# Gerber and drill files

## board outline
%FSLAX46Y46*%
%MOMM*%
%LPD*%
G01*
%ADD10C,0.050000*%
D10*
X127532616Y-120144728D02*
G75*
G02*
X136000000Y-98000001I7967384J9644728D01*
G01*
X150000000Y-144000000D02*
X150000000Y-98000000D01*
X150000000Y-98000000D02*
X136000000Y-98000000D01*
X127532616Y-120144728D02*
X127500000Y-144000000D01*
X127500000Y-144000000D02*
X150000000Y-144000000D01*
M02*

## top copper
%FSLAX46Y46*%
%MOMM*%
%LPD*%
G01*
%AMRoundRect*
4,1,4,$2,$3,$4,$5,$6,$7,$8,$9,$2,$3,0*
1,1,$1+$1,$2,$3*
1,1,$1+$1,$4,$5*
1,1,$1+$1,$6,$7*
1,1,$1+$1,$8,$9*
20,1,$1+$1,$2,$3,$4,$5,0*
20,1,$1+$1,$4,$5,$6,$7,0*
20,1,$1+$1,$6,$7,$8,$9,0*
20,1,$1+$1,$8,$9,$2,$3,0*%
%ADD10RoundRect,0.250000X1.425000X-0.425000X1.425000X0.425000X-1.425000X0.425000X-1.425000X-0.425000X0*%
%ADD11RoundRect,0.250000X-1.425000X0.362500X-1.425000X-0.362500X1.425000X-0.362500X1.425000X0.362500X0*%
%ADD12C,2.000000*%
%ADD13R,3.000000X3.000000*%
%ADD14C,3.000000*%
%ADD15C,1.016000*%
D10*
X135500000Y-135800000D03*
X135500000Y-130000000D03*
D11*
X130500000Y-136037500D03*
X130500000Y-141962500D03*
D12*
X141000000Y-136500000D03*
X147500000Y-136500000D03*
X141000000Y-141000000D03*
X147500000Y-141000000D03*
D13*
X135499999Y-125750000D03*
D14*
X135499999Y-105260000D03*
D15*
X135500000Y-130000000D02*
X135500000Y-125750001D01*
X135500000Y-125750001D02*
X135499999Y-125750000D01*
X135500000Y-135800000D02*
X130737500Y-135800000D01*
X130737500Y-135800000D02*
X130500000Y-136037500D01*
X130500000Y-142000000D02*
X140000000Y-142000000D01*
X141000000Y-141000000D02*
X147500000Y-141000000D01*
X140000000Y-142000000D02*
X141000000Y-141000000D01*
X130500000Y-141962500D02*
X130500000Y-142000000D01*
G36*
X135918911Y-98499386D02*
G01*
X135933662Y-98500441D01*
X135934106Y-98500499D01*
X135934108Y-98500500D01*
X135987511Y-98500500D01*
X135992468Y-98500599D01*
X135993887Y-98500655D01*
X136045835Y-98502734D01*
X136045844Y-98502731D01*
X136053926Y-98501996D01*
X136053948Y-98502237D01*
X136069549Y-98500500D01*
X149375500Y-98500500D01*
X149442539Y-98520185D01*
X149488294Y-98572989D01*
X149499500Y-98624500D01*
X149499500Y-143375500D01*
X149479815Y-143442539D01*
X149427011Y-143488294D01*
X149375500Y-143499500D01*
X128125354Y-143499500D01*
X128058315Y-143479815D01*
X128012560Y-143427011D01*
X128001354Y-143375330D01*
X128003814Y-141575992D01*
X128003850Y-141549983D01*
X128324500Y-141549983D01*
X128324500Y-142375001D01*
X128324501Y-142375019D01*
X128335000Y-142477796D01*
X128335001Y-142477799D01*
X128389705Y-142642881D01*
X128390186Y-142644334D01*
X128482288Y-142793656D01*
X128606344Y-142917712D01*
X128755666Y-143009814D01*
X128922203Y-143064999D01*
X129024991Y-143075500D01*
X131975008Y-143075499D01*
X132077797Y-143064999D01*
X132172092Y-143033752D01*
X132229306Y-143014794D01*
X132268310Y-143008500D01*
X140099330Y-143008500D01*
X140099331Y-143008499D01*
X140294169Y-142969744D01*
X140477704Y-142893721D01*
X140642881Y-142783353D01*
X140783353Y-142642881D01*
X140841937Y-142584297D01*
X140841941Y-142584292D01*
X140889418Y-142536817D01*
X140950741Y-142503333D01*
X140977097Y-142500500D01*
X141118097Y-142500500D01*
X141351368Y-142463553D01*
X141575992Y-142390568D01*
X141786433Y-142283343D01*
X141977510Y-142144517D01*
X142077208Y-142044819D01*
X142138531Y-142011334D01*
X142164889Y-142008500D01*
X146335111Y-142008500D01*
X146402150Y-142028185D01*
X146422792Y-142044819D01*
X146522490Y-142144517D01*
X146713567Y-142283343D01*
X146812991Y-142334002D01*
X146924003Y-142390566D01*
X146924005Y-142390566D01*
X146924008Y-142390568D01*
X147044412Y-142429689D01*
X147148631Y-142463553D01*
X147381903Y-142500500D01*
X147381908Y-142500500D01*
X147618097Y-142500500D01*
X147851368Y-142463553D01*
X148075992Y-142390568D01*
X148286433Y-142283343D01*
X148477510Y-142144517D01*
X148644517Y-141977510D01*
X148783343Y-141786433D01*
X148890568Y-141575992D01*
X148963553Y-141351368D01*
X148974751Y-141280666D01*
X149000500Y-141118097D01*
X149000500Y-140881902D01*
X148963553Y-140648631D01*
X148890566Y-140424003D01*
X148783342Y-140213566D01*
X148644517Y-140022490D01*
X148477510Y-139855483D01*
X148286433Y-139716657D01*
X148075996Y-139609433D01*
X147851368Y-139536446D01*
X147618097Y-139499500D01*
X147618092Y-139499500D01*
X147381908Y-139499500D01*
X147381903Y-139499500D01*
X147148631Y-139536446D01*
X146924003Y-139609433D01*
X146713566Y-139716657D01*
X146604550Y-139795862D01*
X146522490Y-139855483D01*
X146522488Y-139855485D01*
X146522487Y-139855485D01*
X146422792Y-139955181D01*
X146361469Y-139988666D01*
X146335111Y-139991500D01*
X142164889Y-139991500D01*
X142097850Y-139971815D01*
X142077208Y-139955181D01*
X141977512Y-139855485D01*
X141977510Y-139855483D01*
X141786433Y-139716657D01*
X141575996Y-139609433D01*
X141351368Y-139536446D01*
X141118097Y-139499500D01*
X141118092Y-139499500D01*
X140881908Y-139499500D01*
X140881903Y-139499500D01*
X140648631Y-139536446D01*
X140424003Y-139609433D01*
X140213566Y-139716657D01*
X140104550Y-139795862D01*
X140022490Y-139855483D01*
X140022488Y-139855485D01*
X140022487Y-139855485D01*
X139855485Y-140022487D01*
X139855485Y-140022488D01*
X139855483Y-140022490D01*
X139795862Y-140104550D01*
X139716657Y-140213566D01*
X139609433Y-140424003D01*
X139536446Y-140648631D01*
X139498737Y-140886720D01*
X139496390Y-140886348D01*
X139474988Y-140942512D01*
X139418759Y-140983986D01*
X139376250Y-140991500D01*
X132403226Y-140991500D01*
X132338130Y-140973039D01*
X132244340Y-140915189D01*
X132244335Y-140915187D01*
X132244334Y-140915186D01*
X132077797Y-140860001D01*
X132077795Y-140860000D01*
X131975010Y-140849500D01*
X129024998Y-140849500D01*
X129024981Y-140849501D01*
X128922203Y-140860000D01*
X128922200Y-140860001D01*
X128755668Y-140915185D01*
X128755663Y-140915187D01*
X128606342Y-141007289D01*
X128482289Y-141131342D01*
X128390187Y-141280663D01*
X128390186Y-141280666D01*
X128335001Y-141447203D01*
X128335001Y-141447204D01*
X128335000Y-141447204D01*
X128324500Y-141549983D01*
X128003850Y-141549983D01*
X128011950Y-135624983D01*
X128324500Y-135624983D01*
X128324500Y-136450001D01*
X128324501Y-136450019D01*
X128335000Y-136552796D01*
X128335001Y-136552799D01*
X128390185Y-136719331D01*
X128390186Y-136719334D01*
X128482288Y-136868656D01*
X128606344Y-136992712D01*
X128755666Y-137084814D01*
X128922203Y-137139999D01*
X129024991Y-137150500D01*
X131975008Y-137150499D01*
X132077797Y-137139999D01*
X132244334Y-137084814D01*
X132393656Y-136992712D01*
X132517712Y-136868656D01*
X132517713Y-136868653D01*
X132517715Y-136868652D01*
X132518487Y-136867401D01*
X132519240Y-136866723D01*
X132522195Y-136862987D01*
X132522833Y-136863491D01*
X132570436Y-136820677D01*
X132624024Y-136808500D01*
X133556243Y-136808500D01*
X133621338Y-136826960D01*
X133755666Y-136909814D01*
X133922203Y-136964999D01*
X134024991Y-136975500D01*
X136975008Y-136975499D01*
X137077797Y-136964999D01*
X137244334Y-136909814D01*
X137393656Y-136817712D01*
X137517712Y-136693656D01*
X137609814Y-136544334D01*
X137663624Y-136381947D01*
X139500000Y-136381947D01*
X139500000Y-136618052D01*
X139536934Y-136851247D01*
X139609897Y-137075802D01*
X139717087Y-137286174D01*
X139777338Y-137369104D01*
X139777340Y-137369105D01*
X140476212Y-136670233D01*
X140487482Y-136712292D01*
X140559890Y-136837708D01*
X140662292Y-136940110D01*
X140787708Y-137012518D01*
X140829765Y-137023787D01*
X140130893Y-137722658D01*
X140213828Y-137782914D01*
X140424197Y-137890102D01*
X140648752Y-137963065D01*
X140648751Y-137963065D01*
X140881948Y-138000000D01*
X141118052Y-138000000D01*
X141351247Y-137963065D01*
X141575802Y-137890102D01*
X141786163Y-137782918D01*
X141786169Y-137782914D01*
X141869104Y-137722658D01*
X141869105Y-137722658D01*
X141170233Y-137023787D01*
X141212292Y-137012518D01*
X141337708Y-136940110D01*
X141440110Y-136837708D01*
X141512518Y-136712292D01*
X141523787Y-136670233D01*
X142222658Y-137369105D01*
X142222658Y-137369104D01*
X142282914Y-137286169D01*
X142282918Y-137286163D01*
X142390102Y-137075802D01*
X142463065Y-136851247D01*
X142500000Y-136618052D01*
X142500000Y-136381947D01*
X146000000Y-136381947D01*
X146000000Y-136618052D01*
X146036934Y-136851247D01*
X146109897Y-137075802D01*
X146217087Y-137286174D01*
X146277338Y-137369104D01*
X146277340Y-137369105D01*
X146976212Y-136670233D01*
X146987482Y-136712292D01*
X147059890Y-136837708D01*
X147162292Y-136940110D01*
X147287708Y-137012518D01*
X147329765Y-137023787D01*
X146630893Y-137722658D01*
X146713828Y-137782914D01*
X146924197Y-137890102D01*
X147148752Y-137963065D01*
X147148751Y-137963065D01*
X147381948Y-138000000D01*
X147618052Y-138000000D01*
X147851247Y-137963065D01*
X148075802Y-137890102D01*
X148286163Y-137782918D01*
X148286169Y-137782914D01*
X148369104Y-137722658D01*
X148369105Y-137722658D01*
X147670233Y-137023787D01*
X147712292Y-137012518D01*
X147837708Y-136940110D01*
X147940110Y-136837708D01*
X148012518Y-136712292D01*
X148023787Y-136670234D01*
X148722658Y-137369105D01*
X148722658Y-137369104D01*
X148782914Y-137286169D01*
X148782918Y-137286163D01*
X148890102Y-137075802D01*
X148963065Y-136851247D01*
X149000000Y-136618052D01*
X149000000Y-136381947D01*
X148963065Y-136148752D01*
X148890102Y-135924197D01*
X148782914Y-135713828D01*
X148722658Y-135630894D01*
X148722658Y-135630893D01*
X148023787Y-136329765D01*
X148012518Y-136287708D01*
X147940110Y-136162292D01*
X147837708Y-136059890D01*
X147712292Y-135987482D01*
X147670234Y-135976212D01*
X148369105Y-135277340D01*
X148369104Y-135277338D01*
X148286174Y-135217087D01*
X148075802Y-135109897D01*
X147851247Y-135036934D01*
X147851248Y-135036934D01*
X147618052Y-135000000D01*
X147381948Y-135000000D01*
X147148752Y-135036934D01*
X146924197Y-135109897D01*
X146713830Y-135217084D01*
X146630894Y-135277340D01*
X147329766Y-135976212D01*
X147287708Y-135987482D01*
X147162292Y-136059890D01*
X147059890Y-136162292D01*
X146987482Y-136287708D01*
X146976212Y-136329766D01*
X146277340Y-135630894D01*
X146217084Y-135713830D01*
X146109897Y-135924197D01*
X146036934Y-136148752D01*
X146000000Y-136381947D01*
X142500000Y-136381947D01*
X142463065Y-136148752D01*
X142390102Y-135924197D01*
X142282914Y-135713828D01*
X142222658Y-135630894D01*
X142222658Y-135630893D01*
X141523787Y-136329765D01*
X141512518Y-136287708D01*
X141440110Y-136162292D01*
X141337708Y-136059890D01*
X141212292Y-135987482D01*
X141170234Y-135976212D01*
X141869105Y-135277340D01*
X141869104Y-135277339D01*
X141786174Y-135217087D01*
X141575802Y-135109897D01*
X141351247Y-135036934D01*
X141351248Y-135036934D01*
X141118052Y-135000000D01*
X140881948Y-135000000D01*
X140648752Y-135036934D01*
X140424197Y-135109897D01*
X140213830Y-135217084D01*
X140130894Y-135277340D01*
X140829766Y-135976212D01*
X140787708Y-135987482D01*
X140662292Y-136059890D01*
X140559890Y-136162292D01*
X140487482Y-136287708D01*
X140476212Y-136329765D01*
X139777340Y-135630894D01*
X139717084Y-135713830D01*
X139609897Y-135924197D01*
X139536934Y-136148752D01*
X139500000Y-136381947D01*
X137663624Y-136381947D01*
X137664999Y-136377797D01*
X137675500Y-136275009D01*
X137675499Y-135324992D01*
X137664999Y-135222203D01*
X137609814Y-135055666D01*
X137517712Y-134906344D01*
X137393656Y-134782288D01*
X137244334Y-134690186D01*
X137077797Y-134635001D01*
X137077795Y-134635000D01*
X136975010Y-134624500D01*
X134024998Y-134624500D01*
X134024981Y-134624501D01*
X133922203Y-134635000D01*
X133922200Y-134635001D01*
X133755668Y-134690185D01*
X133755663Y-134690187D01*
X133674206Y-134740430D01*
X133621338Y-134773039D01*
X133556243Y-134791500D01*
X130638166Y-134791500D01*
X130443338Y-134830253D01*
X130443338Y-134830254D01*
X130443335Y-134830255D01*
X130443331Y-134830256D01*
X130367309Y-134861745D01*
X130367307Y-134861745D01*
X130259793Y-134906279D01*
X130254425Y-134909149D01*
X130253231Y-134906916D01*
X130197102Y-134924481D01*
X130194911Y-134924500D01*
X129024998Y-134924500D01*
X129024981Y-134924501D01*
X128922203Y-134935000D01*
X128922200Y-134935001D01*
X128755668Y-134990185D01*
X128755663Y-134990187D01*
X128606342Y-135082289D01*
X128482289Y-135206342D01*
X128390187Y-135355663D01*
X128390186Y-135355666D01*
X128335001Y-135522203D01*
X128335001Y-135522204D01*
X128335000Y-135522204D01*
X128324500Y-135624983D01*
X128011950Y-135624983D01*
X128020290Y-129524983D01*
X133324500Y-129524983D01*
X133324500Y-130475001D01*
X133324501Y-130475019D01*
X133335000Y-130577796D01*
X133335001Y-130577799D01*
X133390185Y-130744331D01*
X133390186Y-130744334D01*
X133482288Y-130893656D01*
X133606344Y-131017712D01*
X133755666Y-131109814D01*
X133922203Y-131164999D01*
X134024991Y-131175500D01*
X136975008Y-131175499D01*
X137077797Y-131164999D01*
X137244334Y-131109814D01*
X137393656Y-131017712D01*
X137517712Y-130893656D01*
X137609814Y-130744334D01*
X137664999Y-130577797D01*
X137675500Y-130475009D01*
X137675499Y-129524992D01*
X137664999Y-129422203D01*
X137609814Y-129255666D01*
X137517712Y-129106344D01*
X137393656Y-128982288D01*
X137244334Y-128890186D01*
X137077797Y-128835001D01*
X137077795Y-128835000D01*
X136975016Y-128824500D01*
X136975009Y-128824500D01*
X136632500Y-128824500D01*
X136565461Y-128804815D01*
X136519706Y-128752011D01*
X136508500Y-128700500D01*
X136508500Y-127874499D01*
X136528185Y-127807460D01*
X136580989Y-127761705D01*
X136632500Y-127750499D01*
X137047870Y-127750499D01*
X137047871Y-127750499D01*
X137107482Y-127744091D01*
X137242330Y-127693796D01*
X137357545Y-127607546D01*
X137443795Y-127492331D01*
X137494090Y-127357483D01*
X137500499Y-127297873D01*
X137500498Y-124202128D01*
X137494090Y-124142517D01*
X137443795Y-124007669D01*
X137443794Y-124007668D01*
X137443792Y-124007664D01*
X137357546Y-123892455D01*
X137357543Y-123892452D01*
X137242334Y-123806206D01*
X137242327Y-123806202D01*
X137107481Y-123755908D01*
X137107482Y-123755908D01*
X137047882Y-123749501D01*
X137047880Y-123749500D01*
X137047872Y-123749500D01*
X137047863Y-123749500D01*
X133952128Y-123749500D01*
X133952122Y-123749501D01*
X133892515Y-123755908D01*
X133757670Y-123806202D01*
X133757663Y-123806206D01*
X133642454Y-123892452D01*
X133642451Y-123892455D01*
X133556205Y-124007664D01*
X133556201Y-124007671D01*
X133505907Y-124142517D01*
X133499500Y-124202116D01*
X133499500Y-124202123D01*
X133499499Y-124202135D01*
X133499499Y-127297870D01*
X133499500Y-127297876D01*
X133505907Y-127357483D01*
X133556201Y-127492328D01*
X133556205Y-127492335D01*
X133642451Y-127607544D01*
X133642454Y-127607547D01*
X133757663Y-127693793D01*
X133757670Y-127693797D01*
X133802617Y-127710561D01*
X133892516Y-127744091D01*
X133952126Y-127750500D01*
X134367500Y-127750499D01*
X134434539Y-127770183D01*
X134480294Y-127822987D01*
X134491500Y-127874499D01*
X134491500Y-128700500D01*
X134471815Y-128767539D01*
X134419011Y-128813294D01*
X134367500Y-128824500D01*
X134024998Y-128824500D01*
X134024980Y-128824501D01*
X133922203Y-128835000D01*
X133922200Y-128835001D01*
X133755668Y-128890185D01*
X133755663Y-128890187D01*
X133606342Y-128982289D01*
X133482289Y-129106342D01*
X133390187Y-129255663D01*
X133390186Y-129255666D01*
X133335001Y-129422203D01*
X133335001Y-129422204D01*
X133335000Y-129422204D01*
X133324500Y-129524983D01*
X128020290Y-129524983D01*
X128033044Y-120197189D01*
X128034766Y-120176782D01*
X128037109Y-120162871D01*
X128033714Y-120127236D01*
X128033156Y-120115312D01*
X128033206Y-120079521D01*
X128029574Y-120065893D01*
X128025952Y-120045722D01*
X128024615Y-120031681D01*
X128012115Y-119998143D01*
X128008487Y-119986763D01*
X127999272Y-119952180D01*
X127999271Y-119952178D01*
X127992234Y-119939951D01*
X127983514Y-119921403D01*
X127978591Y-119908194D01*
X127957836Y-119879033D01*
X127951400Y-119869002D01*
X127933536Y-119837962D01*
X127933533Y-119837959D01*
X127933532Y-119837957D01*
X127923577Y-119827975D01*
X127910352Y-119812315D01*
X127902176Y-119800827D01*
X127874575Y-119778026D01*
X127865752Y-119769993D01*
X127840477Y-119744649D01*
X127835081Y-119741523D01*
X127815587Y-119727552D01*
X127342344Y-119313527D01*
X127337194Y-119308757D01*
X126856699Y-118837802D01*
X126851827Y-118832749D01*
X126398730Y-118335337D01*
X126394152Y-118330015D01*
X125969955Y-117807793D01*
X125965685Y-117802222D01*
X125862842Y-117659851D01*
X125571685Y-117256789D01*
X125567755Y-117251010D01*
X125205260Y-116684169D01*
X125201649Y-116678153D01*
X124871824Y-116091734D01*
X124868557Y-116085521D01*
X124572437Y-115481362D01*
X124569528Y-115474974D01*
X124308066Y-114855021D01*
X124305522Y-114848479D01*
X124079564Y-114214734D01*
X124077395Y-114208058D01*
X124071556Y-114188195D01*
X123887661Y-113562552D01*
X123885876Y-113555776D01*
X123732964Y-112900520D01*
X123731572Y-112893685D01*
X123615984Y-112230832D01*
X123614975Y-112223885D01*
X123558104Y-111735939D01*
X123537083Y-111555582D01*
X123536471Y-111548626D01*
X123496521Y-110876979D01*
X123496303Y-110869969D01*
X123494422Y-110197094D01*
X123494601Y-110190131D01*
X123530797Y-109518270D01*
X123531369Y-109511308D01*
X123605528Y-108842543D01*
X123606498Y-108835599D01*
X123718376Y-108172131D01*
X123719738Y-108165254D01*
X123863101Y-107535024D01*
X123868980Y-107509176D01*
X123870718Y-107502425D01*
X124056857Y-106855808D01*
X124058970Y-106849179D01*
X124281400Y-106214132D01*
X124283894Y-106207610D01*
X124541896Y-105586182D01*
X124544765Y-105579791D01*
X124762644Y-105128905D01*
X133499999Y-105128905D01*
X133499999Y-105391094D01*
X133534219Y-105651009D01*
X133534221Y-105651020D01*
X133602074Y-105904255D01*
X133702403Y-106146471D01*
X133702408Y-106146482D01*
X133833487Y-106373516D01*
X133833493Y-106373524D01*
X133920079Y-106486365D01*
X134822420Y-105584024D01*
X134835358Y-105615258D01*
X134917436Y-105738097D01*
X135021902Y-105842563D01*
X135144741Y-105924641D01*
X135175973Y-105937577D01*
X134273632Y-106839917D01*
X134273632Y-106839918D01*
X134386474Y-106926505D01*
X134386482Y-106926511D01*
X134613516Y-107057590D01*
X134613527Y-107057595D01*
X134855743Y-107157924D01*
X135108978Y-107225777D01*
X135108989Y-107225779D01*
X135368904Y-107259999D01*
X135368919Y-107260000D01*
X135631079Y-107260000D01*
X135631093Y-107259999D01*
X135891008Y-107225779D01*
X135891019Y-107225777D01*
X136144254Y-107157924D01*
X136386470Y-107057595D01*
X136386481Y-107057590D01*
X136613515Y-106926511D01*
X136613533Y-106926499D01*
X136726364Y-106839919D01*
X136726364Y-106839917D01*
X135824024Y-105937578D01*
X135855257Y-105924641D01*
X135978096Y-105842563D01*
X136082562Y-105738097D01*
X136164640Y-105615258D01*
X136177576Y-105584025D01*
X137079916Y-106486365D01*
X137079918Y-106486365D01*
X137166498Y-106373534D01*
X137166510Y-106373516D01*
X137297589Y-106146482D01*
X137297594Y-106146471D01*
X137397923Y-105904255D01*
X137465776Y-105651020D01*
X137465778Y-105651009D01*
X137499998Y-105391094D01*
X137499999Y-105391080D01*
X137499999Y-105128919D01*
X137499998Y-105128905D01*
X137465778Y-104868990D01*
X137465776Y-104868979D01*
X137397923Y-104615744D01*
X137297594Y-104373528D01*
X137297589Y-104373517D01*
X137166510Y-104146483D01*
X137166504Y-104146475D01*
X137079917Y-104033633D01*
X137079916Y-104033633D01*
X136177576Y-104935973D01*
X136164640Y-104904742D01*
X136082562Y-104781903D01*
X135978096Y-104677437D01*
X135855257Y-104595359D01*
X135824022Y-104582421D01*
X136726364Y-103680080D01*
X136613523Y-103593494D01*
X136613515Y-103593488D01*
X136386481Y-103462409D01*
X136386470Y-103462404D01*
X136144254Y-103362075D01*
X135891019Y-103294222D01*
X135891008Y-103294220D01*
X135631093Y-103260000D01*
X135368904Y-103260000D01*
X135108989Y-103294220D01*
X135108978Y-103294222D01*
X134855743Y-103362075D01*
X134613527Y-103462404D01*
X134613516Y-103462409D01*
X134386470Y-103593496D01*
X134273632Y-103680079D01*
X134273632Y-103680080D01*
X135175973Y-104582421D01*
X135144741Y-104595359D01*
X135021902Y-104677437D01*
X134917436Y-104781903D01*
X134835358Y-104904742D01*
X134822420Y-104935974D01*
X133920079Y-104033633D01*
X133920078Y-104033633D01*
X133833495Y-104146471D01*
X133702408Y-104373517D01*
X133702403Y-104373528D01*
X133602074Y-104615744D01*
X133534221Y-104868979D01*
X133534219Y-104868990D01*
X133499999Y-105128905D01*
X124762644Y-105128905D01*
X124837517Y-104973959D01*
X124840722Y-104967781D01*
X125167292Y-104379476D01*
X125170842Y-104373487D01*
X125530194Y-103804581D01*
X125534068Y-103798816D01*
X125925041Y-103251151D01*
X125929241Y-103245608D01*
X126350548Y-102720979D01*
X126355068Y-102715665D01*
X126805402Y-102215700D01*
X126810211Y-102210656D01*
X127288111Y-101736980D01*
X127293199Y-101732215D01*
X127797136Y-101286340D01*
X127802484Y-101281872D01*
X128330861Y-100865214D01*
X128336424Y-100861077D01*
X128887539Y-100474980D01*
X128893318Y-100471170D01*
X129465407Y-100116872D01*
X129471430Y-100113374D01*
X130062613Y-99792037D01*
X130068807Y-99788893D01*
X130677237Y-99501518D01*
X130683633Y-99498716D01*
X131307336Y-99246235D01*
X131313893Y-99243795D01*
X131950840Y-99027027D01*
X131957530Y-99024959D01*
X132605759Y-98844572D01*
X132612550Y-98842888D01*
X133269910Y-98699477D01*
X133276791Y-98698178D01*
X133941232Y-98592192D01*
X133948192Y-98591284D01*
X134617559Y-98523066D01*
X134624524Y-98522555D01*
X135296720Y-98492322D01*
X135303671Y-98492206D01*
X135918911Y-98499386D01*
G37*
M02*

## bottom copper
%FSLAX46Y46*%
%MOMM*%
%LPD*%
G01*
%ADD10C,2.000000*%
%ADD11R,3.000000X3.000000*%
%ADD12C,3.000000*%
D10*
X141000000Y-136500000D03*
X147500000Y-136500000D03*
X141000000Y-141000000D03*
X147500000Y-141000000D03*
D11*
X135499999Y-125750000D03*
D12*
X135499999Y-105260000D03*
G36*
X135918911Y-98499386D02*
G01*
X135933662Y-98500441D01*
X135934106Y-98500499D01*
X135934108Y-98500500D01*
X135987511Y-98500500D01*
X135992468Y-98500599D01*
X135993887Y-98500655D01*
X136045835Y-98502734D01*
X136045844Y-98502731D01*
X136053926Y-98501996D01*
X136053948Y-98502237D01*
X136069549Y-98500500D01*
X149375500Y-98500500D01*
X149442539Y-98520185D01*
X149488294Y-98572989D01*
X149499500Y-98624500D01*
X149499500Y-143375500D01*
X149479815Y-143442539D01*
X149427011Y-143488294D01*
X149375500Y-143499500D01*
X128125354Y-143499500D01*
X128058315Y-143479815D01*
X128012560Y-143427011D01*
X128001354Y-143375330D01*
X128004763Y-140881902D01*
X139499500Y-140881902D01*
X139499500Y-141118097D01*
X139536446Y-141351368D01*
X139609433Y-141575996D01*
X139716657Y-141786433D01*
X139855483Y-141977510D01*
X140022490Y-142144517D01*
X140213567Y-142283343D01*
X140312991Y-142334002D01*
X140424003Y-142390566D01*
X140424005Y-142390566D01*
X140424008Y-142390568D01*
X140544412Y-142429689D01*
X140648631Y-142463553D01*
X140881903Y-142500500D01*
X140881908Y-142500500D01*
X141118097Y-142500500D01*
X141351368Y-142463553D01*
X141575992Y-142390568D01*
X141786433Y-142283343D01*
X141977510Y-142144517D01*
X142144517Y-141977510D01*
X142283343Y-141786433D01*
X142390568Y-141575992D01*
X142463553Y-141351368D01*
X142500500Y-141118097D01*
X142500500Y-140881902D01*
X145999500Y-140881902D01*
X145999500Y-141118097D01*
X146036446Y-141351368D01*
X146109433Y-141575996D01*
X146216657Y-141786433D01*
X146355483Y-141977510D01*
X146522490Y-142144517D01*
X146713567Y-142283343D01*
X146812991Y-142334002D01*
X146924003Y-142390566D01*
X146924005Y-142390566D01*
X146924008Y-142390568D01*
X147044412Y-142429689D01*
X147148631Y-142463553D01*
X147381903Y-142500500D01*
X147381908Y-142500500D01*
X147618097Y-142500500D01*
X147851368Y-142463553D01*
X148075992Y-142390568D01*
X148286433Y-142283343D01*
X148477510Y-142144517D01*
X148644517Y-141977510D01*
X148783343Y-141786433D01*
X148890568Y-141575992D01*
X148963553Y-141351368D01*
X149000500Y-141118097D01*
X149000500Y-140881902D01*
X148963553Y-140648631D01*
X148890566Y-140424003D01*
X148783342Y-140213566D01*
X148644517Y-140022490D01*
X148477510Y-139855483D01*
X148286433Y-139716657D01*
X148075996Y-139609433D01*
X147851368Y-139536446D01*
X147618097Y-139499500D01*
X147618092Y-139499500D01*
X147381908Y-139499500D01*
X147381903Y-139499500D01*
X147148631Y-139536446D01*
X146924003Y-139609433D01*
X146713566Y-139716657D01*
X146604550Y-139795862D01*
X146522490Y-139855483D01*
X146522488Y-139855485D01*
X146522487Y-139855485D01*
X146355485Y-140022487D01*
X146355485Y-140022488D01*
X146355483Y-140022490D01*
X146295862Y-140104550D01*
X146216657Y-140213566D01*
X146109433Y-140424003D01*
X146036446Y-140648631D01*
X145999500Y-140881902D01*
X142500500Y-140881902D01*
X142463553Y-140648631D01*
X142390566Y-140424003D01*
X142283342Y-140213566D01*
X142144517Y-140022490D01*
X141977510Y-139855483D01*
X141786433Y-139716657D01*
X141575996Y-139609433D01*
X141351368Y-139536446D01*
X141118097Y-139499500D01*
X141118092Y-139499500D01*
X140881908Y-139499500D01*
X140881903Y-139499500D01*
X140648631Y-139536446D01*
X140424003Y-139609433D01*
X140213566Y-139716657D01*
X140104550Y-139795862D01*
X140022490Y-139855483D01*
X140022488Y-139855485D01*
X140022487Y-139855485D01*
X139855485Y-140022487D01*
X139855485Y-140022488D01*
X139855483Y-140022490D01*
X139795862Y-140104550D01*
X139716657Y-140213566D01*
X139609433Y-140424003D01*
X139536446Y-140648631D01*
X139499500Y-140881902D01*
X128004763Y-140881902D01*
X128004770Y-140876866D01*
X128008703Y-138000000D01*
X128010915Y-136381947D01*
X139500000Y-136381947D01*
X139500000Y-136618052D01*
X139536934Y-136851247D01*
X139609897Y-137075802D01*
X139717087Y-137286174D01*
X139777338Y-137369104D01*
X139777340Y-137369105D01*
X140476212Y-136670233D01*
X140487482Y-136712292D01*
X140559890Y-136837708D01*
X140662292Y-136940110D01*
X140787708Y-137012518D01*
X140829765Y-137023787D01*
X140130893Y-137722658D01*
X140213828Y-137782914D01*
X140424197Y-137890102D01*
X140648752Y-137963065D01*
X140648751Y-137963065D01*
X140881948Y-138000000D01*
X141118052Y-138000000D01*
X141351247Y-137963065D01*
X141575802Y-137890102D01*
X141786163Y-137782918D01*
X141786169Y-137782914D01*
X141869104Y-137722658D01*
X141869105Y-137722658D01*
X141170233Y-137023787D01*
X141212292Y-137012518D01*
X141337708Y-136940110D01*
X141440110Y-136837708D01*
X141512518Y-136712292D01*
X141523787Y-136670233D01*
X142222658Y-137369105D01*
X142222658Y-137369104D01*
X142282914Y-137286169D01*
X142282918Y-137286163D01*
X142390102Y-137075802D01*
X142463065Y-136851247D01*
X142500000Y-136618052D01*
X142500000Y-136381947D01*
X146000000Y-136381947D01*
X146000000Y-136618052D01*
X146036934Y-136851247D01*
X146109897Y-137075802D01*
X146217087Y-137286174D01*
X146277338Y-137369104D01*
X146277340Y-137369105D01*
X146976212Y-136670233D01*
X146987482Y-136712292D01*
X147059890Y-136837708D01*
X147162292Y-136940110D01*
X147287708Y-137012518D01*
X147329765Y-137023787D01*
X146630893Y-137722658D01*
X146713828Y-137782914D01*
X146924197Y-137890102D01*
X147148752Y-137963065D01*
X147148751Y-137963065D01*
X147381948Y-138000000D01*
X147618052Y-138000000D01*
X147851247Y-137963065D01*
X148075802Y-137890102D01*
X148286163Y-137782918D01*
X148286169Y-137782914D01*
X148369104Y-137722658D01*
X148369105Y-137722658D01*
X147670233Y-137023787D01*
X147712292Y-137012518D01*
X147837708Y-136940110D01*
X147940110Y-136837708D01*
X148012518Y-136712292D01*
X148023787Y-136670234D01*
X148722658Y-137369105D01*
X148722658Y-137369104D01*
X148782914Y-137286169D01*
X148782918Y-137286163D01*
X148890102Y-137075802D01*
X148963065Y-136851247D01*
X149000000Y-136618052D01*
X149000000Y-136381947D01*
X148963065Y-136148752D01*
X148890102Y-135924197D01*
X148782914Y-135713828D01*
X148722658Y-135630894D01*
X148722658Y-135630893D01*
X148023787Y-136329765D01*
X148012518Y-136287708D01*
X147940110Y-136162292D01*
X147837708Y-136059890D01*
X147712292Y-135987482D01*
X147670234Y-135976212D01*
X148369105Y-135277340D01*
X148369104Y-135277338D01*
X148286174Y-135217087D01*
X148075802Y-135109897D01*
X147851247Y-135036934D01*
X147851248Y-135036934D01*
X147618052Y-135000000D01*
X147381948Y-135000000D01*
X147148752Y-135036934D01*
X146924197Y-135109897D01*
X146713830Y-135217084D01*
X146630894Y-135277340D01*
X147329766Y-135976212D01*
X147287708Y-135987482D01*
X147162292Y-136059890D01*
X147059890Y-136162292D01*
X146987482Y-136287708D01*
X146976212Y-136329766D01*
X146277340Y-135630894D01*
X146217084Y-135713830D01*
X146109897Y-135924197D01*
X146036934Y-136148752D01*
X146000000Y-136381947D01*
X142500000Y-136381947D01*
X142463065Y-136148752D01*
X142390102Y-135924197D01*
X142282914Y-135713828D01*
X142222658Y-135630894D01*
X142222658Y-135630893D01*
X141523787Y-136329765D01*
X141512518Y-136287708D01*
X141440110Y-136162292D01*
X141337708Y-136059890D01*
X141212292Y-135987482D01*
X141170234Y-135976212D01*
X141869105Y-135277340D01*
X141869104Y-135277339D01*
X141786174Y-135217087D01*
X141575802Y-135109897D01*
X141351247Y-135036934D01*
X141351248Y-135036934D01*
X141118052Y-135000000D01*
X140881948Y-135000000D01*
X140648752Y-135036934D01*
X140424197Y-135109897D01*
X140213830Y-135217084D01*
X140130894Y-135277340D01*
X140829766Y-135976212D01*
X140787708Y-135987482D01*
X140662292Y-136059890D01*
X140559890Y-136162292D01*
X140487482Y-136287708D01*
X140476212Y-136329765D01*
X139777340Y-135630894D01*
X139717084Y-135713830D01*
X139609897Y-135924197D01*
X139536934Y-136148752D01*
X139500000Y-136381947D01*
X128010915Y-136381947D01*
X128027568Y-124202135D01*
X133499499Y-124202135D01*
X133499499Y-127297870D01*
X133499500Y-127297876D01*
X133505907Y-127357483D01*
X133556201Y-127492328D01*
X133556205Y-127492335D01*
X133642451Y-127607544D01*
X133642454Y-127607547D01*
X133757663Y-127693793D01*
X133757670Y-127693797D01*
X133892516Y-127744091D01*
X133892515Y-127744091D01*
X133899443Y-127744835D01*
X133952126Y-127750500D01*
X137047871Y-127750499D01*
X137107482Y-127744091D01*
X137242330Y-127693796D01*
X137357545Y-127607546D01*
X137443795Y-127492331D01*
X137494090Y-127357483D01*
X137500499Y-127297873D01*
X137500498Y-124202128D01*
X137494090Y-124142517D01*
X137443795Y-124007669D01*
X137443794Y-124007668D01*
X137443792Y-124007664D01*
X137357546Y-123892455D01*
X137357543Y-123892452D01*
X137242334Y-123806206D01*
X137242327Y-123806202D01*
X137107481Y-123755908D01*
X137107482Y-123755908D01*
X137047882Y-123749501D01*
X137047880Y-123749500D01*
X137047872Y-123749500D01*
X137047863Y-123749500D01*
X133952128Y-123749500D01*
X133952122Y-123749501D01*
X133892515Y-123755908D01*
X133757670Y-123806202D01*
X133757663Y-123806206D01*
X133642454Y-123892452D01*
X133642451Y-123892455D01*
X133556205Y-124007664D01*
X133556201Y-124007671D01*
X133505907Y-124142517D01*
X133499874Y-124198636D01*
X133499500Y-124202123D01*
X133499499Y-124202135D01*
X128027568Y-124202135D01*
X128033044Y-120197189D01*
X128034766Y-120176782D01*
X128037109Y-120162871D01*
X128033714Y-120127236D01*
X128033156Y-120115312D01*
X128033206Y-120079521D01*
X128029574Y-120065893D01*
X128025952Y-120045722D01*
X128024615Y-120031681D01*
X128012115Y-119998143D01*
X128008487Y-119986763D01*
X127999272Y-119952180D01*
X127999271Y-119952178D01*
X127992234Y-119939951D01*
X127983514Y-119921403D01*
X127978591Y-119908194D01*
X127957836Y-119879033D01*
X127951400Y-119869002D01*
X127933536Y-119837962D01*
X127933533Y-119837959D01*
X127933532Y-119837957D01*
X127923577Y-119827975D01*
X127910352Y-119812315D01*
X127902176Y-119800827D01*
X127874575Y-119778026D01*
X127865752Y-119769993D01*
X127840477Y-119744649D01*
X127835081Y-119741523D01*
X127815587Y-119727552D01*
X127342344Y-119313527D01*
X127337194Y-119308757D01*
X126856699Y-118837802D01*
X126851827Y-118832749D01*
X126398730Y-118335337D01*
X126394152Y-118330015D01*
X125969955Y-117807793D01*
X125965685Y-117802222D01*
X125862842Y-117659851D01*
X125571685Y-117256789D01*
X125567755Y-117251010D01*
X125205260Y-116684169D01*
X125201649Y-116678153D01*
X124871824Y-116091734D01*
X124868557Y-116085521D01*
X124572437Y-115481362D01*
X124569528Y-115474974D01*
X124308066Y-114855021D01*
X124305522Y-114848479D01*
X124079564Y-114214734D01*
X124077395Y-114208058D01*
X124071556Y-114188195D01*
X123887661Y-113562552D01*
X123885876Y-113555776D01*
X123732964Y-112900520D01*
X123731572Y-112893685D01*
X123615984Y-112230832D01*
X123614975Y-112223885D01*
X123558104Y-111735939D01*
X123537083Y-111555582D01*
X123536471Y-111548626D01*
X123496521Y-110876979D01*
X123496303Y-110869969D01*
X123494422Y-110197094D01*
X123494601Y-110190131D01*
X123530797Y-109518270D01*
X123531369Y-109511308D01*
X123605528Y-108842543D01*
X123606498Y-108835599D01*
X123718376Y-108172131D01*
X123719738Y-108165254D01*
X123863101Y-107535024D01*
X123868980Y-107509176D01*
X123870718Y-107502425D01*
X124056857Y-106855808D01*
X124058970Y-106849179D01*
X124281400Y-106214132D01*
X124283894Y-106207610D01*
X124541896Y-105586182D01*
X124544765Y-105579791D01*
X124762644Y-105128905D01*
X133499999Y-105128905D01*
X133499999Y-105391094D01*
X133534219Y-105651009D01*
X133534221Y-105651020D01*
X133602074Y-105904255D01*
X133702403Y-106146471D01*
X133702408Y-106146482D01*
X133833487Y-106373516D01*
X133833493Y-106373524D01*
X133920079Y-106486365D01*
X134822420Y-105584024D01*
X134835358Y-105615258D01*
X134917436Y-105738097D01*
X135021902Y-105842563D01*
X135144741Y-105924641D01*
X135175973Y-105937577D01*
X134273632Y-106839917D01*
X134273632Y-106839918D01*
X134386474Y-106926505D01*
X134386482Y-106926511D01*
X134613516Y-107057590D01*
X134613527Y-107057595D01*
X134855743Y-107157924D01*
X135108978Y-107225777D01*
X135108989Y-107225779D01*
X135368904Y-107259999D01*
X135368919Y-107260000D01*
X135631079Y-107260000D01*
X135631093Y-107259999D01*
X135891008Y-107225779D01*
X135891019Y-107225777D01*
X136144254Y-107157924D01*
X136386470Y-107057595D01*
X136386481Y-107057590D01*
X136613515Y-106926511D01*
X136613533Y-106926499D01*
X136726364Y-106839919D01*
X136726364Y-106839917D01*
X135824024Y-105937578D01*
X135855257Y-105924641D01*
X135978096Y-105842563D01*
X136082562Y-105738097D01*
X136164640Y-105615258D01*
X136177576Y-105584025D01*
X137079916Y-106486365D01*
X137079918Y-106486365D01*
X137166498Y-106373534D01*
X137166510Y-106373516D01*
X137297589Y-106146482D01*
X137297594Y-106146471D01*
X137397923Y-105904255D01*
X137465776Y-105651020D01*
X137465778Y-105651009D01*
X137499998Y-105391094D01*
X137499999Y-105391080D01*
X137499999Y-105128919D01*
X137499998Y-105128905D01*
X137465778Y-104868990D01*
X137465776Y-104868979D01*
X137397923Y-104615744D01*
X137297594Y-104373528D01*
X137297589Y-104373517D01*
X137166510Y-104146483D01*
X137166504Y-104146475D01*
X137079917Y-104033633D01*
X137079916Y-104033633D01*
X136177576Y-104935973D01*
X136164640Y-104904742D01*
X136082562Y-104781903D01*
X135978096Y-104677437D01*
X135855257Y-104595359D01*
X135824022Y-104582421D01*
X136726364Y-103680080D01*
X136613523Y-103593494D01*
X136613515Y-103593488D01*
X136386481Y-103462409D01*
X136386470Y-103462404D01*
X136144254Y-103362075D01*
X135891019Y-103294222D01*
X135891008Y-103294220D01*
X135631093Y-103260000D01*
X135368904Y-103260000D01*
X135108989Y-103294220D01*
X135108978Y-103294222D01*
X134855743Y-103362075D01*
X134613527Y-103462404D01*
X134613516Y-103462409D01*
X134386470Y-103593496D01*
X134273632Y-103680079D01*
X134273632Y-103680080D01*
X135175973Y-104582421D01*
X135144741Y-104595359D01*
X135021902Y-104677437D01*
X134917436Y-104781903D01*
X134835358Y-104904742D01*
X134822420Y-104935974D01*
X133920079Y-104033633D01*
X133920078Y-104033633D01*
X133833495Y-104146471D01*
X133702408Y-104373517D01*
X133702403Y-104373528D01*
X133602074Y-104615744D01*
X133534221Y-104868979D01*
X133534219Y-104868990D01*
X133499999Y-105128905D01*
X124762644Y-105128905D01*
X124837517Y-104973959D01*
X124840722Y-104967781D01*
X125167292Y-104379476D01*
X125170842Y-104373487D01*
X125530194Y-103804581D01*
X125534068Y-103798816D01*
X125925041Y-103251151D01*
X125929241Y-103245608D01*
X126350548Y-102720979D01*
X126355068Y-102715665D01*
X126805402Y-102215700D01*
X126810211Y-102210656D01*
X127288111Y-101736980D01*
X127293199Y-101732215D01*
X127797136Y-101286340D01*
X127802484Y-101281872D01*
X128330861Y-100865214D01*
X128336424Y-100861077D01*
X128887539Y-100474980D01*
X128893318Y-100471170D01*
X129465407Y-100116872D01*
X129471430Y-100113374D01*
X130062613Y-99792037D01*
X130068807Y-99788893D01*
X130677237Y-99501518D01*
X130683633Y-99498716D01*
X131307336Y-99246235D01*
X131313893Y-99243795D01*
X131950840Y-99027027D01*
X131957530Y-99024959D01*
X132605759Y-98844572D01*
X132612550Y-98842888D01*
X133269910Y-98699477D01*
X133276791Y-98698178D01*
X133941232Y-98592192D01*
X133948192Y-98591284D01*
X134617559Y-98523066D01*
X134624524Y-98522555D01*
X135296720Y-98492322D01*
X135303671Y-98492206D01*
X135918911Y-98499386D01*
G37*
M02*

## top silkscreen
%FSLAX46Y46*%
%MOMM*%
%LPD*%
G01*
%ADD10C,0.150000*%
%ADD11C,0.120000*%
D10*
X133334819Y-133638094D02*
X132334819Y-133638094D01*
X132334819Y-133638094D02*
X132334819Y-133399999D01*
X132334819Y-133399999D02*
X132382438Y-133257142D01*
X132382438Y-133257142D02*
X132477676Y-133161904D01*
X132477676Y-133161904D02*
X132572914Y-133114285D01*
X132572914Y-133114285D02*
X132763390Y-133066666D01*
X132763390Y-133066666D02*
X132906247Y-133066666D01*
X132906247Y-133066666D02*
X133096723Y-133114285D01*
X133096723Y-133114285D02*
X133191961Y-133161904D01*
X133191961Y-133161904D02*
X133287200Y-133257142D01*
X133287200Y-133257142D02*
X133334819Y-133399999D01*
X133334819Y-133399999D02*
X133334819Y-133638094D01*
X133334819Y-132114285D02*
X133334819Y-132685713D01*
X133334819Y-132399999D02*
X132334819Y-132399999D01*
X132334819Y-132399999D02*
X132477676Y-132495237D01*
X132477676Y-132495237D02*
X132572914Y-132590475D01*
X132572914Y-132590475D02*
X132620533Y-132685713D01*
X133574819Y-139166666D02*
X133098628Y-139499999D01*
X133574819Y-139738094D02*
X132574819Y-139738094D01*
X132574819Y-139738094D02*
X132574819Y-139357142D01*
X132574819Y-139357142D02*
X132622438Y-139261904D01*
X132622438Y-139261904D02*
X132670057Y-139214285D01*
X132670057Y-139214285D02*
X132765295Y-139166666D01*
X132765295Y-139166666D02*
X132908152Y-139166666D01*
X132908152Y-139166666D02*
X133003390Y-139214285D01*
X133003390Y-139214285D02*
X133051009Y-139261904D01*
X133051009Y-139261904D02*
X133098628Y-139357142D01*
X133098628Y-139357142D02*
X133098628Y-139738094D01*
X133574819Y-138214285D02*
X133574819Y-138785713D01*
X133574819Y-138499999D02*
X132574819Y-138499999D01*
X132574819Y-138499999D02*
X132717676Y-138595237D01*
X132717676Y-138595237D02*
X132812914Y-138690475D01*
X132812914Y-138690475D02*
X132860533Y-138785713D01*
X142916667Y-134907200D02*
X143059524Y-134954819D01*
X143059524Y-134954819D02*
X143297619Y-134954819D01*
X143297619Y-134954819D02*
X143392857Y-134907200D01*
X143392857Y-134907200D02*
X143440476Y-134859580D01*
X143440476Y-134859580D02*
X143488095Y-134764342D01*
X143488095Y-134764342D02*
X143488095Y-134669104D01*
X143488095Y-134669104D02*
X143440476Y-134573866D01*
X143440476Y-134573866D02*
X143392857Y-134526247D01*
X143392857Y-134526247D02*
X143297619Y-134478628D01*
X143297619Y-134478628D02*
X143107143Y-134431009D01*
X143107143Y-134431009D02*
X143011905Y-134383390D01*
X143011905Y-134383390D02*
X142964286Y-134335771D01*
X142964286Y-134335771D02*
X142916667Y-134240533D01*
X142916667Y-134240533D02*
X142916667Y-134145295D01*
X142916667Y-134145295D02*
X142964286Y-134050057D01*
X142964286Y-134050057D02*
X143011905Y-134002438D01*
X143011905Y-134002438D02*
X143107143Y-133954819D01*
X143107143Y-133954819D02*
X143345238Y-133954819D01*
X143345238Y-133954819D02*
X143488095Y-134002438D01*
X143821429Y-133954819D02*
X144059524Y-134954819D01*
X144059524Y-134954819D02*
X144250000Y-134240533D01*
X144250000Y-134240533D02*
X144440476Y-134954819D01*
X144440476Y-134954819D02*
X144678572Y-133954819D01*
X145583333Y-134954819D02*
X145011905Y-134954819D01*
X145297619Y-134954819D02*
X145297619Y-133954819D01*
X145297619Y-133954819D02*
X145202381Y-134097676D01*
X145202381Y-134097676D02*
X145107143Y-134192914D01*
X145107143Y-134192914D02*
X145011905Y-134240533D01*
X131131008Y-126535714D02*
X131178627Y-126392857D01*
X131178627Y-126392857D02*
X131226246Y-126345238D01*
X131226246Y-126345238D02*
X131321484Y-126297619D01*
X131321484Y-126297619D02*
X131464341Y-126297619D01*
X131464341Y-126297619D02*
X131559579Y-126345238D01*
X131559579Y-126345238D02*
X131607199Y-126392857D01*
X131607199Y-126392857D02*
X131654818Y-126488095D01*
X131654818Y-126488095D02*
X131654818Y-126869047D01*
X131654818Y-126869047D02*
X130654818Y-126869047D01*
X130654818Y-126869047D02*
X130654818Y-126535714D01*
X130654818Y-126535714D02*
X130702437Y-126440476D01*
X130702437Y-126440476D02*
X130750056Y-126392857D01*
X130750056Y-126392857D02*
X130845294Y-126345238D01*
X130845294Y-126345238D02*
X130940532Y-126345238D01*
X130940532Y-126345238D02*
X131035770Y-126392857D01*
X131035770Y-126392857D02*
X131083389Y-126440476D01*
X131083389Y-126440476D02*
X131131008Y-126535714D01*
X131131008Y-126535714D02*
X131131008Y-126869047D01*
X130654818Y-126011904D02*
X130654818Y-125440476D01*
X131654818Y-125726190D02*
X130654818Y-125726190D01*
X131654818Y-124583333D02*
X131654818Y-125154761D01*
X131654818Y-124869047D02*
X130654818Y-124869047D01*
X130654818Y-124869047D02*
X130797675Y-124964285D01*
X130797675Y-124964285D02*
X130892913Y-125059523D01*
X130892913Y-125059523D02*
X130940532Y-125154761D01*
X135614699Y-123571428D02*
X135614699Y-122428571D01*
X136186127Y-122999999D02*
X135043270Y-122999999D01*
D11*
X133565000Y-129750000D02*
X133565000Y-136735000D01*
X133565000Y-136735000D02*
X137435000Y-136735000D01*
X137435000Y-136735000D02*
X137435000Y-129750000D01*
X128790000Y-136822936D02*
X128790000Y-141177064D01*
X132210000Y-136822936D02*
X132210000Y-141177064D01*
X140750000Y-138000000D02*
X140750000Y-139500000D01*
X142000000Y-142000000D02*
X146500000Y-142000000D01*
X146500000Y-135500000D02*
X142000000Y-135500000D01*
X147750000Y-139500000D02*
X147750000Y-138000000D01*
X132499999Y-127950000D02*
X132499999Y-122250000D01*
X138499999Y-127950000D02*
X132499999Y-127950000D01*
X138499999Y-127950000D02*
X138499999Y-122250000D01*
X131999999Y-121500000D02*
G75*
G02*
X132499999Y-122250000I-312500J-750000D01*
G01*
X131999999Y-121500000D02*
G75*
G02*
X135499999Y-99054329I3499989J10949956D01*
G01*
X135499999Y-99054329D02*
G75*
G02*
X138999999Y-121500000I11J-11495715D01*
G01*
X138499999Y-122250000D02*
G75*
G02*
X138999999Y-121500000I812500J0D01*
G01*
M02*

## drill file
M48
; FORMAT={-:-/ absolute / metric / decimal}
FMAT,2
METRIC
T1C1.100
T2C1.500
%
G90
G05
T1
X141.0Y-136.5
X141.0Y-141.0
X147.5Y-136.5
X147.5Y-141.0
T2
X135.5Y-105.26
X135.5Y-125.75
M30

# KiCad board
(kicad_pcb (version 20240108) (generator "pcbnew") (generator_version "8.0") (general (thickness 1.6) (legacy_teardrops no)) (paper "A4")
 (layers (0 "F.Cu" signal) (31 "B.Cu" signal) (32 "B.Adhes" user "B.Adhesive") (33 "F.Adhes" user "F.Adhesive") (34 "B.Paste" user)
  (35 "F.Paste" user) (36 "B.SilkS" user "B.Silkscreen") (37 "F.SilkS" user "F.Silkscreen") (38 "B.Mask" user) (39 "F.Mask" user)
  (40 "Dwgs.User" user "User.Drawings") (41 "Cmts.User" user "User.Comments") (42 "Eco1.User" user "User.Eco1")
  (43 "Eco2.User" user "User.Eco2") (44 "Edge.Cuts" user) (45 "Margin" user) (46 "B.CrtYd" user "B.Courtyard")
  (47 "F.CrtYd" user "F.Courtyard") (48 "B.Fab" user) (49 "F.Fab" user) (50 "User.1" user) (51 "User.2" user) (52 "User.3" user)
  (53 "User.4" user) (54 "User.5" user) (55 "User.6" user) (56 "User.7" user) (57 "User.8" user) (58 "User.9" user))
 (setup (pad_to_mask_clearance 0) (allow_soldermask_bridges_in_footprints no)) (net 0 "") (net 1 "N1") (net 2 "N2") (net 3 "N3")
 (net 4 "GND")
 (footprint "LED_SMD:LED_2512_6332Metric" (layer "F.Cu") (at 135.5 132.9 90)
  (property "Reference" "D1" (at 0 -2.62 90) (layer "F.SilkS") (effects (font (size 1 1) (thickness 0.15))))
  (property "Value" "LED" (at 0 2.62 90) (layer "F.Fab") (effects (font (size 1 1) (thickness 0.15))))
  (fp_line (start 3.15 -1.935) (end -3.835 -1.935) (stroke (width 0.12) (type solid)) (layer "F.SilkS"))
  (fp_line (start -3.835 -1.935) (end -3.835 1.935) (stroke (width 0.12) (type solid)) (layer "F.SilkS"))
  (fp_line (start -3.835 1.935) (end 3.15 1.935) (stroke (width 0.12) (type solid)) (layer "F.SilkS"))
  (pad "1" smd roundrect (at -2.9 0 90) (size 1.35 3.35) (layers "F.Cu" "F.Paste" "F.Mask") (roundrect_rratio 0.185185) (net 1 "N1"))
  (pad "2" smd roundrect (at 2.9 0 90) (size 1.35 3.35) (layers "F.Cu" "F.Paste" "F.Mask") (roundrect_rratio 0.185185) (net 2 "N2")))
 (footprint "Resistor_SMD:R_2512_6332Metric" (layer "F.Cu") (at 130.5 139 -90)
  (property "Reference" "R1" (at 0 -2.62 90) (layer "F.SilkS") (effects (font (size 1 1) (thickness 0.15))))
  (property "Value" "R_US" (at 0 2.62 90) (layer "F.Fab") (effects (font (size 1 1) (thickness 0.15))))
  (fp_line (start -2.177064 1.71) (end 2.177064 1.71) (stroke (width 0.12) (type solid)) (layer "F.SilkS"))
  (fp_line (start -2.177064 -1.71) (end 2.177064 -1.71) (stroke (width 0.12) (type solid)) (layer "F.SilkS"))
  (pad "1" smd roundrect (at -2.9625 0 270) (size 1.225 3.35) (layers "F.Cu" "F.Paste" "F.Mask") (roundrect_rratio 0.204082) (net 1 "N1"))
  (pad "2" smd roundrect (at 2.9625 0 270) (size 1.225 3.35) (layers "F.Cu" "F.Paste" "F.Mask") (roundrect_rratio 0.204082) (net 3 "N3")))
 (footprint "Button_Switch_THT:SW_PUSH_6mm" (layer "F.Cu") (at 141 136.5)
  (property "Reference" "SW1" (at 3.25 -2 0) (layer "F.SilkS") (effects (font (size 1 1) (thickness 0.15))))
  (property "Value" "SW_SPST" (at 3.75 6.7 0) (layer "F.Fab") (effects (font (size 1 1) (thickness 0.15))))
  (fp_line (start -0.25 1.5) (end -0.25 3) (stroke (width 0.12) (type solid)) (layer "F.SilkS"))
  (fp_line (start 1 5.5) (end 5.5 5.5) (stroke (width 0.12) (type solid)) (layer "F.SilkS"))
  (fp_line (start 5.5 -1) (end 1 -1) (stroke (width 0.12) (type solid)) (layer "F.SilkS"))
  (fp_line (start 6.75 3) (end 6.75 1.5) (stroke (width 0.12) (type solid)) (layer "F.SilkS"))
  (pad "1" thru_hole circle (at 0 0 90) (size 2 2) (drill 1.1) (layers "*.Cu" "*.Mask") (remove_unused_layers no) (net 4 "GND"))
  (pad "1" thru_hole circle (at 6.5 0 90) (size 2 2) (drill 1.1) (layers "*.Cu" "*.Mask") (remove_unused_layers no) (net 4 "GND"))
  (pad "2" thru_hole circle (at 0 4.5 90) (size 2 2) (drill 1.1) (layers "*.Cu" "*.Mask") (remove_unused_layers no) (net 3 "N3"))
  (pad "2" thru_hole circle (at 6.5 4.5 90) (size 2 2) (drill 1.1) (layers "*.Cu" "*.Mask") (remove_unused_layers no) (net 3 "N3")))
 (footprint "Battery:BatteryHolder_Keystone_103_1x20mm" (layer "F.Cu") (at 135.499999 125.75 90)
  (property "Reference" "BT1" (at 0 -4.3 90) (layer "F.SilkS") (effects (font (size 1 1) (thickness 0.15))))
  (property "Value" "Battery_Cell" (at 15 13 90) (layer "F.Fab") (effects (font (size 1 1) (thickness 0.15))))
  (fp_line (start -2.2 -3) (end 3.5 -3) (stroke (width 0.12) (type solid)) (layer "F.SilkS"))
  (fp_line (start -2.2 3) (end -2.2 -3) (stroke (width 0.12) (type solid)) (layer "F.SilkS"))
  (fp_line (start -2.2 3) (end 3.5 3) (stroke (width 0.12) (type solid)) (layer "F.SilkS"))
  (fp_arc (start 4.25 -3.5) (mid 3.950694 -3.136459) (end 3.5 -3) (stroke (width 0.12) (type solid)) (layer "F.SilkS"))
  (fp_arc (start 4.25 -3.5) (mid 16.971103 -11.358466) (end 26.695671 0) (stroke (width 0.12) (type solid)) (layer "F.SilkS"))
  (fp_arc (start 26.695671 0) (mid 16.971103 11.358466) (end 4.25 3.5) (stroke (width 0.12) (type solid)) (layer "F.SilkS"))
  (fp_arc (start 3.5 3) (mid 3.950694 3.136459) (end 4.25 3.5) (stroke (width 0.12) (type solid)) (layer "F.SilkS"))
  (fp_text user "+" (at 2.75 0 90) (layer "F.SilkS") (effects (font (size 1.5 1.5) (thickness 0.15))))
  (pad "1" thru_hole rect (at 0 0 90) (size 3 3) (drill 1.5) (layers "*.Cu" "*.Mask") (remove_unused_layers no) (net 2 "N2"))
  (pad "2" thru_hole circle (at 20.49 0 90) (size 3 3) (drill 1.5) (layers "*.Cu" "*.Mask") (remove_unused_layers no) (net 4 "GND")))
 (gr_arc (start 127.532616 120.144728) (mid 123.815065 106.032082) (end 136 98) (stroke (width 0.05) (type default)) (layer "Edge.Cuts"))
 (gr_line (start 150 144) (end 150 98) (stroke (width 0.05) (type default)) (layer "Edge.Cuts"))
 (gr_line (start 150 98) (end 136 98) (stroke (width 0.05) (type default)) (layer "Edge.Cuts"))
 (gr_line (start 127.532616 120.144728) (end 127.5 144) (stroke (width 0.05) (type default)) (layer "Edge.Cuts"))
 (gr_line (start 127.5 144) (end 150 144) (stroke (width 0.05) (type default)) (layer "Edge.Cuts"))
 (segment (start 135.5 130) (end 135.5 125.750001) (width 1.016) (layer "F.Cu") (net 2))
 (segment (start 135.5 125.750001) (end 135.499999 125.75) (width 1.016) (layer "F.Cu") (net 2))
 (segment (start 135.5 135.8) (end 130.7375 135.8) (width 1.016) (layer "F.Cu") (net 1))
 (segment (start 130.7375 135.8) (end 130.5 136.0375) (width 1.016) (layer "F.Cu") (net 1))
 (segment (start 130.5 142) (end 140 142) (width 1.016) (layer "F.Cu") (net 3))
 (segment (start 141 141) (end 147.5 141) (width 1.016) (layer "F.Cu") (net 3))
 (segment (start 140 142) (end 141 141) (width 1.016) (layer "F.Cu") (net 3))
 (segment (start 130.5 141.9625) (end 130.5 142) (width 1.016) (layer "F.Cu") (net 3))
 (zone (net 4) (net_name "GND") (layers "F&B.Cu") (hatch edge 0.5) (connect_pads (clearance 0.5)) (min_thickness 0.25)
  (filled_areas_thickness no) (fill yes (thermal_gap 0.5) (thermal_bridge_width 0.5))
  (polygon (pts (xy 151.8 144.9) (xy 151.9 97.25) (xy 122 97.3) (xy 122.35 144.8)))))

